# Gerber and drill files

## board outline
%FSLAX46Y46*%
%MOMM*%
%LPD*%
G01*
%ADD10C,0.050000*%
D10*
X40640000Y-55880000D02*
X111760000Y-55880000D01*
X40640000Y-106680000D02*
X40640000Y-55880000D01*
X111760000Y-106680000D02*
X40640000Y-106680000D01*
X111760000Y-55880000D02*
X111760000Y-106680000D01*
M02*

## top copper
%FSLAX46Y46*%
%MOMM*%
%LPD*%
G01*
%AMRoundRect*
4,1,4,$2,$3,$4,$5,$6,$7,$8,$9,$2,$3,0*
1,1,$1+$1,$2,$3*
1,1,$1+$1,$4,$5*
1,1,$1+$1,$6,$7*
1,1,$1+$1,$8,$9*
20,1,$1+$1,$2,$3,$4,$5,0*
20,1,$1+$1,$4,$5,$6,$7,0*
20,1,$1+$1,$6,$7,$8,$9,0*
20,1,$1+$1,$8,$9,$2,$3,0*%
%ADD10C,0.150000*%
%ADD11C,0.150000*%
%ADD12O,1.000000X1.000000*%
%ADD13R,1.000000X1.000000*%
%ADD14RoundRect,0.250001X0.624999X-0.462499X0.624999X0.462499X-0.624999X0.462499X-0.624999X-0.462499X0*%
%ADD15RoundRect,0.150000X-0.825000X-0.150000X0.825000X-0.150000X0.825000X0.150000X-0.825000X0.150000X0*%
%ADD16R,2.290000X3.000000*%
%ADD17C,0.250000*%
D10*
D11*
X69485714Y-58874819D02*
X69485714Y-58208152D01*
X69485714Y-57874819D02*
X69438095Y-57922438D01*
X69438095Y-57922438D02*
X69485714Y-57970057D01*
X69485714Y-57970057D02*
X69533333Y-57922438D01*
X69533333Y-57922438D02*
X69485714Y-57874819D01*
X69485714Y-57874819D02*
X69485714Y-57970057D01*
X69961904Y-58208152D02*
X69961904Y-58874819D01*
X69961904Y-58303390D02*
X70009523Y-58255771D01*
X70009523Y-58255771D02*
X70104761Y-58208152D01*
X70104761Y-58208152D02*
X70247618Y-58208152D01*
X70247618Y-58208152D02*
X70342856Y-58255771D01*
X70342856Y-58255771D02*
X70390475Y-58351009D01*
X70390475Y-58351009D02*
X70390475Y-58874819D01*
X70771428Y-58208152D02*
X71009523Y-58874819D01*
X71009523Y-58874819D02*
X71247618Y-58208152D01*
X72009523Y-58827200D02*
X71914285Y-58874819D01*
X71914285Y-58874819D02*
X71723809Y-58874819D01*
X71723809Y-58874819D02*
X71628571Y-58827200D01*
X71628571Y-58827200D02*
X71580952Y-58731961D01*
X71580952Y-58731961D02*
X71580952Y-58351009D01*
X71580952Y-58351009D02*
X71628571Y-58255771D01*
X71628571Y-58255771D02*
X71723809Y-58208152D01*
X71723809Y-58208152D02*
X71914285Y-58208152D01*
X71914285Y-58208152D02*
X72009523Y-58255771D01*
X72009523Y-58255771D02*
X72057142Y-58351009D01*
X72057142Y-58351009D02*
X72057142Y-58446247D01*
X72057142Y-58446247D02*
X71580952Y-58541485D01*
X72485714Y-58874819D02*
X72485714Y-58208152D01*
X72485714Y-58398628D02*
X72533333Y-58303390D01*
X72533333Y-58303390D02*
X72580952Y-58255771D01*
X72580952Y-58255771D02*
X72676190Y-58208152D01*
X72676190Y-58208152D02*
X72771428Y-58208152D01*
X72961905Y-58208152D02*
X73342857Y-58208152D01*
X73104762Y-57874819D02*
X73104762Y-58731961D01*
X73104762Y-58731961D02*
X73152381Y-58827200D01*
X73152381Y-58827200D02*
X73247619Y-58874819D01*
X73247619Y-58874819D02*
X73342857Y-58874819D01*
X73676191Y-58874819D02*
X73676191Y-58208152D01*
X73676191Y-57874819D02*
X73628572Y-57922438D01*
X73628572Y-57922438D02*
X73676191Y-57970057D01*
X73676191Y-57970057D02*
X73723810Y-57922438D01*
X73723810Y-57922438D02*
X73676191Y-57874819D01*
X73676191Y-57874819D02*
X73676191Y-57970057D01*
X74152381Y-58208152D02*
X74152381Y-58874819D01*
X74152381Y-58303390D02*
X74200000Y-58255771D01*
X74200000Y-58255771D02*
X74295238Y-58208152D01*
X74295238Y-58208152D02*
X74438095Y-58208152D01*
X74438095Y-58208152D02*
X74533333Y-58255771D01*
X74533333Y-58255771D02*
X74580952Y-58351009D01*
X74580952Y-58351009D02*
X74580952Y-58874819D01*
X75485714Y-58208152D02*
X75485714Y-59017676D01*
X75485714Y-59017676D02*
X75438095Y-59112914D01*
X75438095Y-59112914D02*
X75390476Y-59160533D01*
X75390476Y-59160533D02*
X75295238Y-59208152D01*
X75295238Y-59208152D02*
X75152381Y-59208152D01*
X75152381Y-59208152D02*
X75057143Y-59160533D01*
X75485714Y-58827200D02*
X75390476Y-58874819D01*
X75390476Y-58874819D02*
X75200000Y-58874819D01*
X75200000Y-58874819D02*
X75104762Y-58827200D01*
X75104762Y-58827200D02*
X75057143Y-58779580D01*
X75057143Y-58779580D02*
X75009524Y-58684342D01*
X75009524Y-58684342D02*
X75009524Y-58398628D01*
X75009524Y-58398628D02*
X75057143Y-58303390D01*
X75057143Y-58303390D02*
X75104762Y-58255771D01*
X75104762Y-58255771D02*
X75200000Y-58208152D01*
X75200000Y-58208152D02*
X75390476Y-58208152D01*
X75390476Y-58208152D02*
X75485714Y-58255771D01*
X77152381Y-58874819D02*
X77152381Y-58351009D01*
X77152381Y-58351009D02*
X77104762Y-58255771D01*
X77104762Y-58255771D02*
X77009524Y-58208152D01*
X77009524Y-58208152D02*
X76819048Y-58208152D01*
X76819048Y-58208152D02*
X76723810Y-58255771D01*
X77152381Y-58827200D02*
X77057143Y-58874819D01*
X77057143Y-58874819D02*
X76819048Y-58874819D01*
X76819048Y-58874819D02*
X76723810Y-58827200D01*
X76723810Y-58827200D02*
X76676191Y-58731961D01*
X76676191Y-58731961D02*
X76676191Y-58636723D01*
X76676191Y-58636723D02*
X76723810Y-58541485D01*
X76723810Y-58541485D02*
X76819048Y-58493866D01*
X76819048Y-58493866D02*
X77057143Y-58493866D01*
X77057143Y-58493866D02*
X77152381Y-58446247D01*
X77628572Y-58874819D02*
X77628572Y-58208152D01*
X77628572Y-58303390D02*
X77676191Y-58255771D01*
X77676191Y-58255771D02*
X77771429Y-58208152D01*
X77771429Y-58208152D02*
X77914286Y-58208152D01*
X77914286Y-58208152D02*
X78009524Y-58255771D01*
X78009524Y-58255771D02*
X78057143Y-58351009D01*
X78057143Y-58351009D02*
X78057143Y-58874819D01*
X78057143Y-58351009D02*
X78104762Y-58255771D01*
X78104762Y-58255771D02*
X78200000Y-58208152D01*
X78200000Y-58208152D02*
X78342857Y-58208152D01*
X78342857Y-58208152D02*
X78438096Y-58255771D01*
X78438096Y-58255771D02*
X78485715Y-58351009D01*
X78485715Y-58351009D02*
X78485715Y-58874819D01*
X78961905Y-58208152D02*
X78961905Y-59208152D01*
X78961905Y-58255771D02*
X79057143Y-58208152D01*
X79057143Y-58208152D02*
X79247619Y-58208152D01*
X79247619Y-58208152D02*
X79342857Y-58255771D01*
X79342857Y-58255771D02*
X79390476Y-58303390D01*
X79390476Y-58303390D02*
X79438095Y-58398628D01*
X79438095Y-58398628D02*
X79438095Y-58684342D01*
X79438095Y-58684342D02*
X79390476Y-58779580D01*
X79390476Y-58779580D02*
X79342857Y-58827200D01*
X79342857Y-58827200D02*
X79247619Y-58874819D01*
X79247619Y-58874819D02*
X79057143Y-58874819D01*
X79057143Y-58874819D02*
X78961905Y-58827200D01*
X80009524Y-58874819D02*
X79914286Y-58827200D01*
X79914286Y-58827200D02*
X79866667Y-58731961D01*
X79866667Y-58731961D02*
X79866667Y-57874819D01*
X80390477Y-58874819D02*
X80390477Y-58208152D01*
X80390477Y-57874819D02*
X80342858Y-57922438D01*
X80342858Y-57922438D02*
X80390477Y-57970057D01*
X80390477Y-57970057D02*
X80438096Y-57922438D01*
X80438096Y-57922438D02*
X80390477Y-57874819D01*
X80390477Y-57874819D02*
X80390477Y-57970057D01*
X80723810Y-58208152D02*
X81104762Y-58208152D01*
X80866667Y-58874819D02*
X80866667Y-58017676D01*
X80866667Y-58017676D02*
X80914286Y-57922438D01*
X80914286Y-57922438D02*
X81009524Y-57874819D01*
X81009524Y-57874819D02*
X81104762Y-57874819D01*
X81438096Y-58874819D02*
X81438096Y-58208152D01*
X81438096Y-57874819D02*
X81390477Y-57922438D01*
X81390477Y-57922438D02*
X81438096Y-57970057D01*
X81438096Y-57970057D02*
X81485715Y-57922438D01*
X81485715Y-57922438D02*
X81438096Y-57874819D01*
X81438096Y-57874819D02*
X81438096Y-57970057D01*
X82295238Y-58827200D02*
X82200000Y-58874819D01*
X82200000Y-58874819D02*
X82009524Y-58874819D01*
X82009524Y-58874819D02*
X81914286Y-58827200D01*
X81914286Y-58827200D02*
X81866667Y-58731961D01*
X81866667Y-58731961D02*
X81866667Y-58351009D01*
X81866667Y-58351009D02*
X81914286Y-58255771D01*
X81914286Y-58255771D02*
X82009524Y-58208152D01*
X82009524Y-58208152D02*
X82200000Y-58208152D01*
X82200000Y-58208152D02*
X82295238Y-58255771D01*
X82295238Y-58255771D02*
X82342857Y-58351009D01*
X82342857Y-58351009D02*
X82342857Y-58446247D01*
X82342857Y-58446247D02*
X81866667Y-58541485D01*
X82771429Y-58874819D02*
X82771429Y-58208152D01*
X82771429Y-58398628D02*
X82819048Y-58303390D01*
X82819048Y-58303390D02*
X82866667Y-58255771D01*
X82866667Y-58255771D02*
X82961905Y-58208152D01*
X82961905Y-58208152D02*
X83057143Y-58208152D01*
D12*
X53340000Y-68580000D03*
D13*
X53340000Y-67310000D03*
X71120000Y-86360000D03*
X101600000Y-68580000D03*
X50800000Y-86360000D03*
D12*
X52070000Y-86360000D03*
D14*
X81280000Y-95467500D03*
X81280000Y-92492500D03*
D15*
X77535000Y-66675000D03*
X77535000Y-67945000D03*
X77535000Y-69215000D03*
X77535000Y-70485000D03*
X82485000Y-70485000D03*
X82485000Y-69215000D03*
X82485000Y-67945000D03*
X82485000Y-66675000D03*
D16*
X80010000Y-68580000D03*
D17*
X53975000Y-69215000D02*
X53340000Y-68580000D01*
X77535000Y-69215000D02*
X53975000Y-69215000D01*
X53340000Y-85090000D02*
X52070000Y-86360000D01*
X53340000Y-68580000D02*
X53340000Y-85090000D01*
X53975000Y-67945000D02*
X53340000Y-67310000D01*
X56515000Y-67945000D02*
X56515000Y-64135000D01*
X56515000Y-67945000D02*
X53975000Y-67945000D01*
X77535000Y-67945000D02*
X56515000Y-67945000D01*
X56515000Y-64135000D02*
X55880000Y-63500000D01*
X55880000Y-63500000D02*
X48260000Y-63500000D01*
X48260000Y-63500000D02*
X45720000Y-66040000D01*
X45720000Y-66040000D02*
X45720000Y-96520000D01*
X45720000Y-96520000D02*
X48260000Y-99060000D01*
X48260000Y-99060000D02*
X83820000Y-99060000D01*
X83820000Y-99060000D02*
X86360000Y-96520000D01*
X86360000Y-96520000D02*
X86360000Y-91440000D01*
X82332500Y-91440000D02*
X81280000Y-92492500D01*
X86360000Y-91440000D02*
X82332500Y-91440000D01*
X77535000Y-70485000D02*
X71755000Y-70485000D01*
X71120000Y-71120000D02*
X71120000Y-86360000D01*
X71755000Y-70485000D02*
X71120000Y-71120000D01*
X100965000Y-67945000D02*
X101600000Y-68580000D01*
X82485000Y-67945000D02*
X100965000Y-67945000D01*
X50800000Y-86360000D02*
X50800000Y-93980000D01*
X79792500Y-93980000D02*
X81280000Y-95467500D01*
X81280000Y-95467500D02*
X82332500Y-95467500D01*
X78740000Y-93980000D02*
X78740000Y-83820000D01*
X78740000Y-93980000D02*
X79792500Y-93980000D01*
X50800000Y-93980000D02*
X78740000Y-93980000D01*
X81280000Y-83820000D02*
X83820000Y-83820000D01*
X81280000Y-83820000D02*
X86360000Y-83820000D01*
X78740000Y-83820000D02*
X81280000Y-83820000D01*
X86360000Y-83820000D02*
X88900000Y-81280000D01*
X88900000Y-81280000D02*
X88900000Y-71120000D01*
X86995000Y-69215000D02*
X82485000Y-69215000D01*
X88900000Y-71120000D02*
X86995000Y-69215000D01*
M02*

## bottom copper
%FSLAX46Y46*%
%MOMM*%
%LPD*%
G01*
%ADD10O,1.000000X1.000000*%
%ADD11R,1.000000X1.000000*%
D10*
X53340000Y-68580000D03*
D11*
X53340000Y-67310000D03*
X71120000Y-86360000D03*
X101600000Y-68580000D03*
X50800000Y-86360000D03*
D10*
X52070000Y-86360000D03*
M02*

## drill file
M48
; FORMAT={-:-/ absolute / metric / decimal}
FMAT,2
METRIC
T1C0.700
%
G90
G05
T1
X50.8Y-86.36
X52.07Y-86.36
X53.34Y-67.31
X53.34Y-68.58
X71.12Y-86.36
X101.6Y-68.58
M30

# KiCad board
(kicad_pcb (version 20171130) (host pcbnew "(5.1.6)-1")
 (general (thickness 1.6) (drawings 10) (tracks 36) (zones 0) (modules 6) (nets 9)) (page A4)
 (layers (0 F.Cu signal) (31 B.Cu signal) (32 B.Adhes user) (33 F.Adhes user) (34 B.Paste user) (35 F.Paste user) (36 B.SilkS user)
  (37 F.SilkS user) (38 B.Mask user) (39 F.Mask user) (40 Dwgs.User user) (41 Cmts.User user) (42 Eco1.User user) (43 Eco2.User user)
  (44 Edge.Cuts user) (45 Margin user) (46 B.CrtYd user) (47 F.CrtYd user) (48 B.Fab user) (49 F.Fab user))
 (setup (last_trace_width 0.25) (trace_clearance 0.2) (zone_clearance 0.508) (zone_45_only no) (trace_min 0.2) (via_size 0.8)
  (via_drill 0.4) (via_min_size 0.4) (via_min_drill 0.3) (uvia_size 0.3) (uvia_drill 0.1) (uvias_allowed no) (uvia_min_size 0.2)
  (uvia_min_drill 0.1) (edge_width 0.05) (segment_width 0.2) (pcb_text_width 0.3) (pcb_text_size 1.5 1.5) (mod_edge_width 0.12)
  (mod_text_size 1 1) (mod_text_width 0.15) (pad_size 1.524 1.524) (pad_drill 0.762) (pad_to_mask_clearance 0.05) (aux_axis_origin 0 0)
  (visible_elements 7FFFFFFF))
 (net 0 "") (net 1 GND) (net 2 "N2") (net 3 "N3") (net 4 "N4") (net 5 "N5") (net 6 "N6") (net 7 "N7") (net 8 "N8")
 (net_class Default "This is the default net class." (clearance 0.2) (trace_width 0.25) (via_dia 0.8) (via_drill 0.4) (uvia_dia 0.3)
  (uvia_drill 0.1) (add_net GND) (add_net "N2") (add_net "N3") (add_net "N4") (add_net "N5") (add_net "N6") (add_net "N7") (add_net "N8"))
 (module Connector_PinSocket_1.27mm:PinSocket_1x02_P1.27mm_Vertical (layer F.Cu) (at 53.34 67.31)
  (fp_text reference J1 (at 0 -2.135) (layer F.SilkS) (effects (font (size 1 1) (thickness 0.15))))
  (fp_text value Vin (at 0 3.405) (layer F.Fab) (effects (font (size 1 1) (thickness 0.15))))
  (pad 2 thru_hole oval (at 0 1.27) (size 1 1) (drill 0.7) (layers *.Cu *.Mask) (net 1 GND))
  (pad 1 thru_hole rect (at 0 0) (size 1 1) (drill 0.7) (layers *.Cu *.Mask) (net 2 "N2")))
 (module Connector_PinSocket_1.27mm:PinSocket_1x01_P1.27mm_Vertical (layer F.Cu) (at 71.12 86.36)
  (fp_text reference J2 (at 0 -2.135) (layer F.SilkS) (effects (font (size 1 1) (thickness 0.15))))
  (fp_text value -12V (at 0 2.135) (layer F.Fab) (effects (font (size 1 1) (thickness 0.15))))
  (pad 1 thru_hole rect (at 0 0) (size 1 1) (drill 0.7) (layers *.Cu *.Mask) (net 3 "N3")))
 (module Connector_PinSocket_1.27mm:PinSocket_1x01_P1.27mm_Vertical (layer F.Cu) (at 101.6 68.58)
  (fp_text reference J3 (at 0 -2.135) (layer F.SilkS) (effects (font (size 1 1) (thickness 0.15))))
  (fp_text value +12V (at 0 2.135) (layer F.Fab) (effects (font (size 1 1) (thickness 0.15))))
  (pad 1 thru_hole rect (at 0 0) (size 1 1) (drill 0.7) (layers *.Cu *.Mask) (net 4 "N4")))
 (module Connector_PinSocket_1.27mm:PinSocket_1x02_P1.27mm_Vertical (layer F.Cu) (at 50.8 86.36 90)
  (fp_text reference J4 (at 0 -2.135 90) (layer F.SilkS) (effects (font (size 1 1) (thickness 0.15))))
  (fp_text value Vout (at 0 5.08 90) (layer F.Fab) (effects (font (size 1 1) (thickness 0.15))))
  (pad 1 thru_hole rect (at 0 0 90) (size 1 1) (drill 0.7) (layers *.Cu *.Mask) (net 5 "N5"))
  (pad 2 thru_hole oval (at 0 1.27 90) (size 1 1) (drill 0.7) (layers *.Cu *.Mask) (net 1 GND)))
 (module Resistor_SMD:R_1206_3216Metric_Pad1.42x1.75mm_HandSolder (layer F.Cu) (at 81.28 93.98 90)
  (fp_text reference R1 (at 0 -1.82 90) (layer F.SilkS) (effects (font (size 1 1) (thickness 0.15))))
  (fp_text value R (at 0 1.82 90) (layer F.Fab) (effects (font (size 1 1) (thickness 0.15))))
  (pad 1 smd roundrect (at -1.4875 0 90) (size 1.425 1.75) (layers F.Cu F.Paste F.Mask) (roundrect_rratio 0.175439) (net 5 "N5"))
  (pad 2 smd roundrect (at 1.4875 0 90) (size 1.425 1.75) (layers F.Cu F.Paste F.Mask) (roundrect_rratio 0.175439) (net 2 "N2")))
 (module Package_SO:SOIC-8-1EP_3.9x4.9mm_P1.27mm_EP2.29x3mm (layer F.Cu) (at 80.01 68.58)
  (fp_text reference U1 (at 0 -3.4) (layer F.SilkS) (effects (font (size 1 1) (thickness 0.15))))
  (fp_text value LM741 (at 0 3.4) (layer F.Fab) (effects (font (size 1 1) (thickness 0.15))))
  (pad 1 smd roundrect (at -2.475 -1.905) (size 1.95 0.6) (layers F.Cu F.Paste F.Mask) (roundrect_rratio 0.25) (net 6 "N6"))
  (pad 2 smd roundrect (at -2.475 -0.635) (size 1.95 0.6) (layers F.Cu F.Paste F.Mask) (roundrect_rratio 0.25) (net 2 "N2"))
  (pad 3 smd roundrect (at -2.475 0.635) (size 1.95 0.6) (layers F.Cu F.Paste F.Mask) (roundrect_rratio 0.25) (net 1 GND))
  (pad 4 smd roundrect (at -2.475 1.905) (size 1.95 0.6) (layers F.Cu F.Paste F.Mask) (roundrect_rratio 0.25) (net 3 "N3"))
  (pad 5 smd roundrect (at 2.475 1.905) (size 1.95 0.6) (layers F.Cu F.Paste F.Mask) (roundrect_rratio 0.25) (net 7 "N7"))
  (pad 6 smd roundrect (at 2.475 0.635) (size 1.95 0.6) (layers F.Cu F.Paste F.Mask) (roundrect_rratio 0.25) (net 5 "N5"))
  (pad 7 smd roundrect (at 2.475 -0.635) (size 1.95 0.6) (layers F.Cu F.Paste F.Mask) (roundrect_rratio 0.25) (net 4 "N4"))
  (pad 8 smd roundrect (at 2.475 -1.905) (size 1.95 0.6) (layers F.Cu F.Paste F.Mask) (roundrect_rratio 0.25) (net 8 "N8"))
  (pad 9 smd rect (at 0 0) (size 2.29 3) (layers F.Cu F.Mask))
  (pad "" smd roundrect (at -0.57 -0.75) (size 0.92 1.21) (layers F.Paste) (roundrect_rratio 0.25))
  (pad "" smd roundrect (at -0.57 0.75) (size 0.92 1.21) (layers F.Paste) (roundrect_rratio 0.25))
  (pad "" smd roundrect (at 0.57 -0.75) (size 0.92 1.21) (layers F.Paste) (roundrect_rratio 0.25))
  (pad "" smd roundrect (at 0.57 0.75) (size 0.92 1.21) (layers F.Paste) (roundrect_rratio 0.25)))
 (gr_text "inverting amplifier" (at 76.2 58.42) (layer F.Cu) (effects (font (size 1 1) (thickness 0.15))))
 (gr_line (start 40.64 55.88) (end 111.76 55.88) (layer Edge.Cuts) (width 0.05))
 (gr_line (start 40.64 106.68) (end 40.64 55.88) (layer Edge.Cuts) (width 0.05))
 (gr_line (start 111.76 106.68) (end 40.64 106.68) (layer Edge.Cuts) (width 0.05))
 (gr_line (start 111.76 55.88) (end 111.76 106.68) (layer Edge.Cuts) (width 0.05))
 (segment (start 53.975 69.215) (end 53.34 68.58) (width 0.25) (layer F.Cu) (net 1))
 (segment (start 77.535 69.215) (end 53.975 69.215) (width 0.25) (layer F.Cu) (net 1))
 (segment (start 53.34 85.09) (end 52.07 86.36) (width 0.25) (layer F.Cu) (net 1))
 (segment (start 53.34 68.58) (end 53.34 85.09) (width 0.25) (layer F.Cu) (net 1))
 (segment (start 53.975 67.945) (end 53.34 67.31) (width 0.25) (layer F.Cu) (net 2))
 (segment (start 56.515 67.945) (end 56.515 64.135) (width 0.25) (layer F.Cu) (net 2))
 (segment (start 56.515 67.945) (end 53.975 67.945) (width 0.25) (layer F.Cu) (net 2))
 (segment (start 77.535 67.945) (end 56.515 67.945) (width 0.25) (layer F.Cu) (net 2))
 (segment (start 56.515 64.135) (end 55.88 63.5) (width 0.25) (layer F.Cu) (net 2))
 (segment (start 55.88 63.5) (end 48.26 63.5) (width 0.25) (layer F.Cu) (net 2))
 (segment (start 48.26 63.5) (end 45.72 66.04) (width 0.25) (layer F.Cu) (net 2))
 (segment (start 45.72 66.04) (end 45.72 96.52) (width 0.25) (layer F.Cu) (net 2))
 (segment (start 45.72 96.52) (end 48.26 99.06) (width 0.25) (layer F.Cu) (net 2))
 (segment (start 48.26 99.06) (end 83.82 99.06) (width 0.25) (layer F.Cu) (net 2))
 (segment (start 83.82 99.06) (end 86.36 96.52) (width 0.25) (layer F.Cu) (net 2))
 (segment (start 86.36 96.52) (end 86.36 91.44) (width 0.25) (layer F.Cu) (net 2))
 (segment (start 82.3325 91.44) (end 81.28 92.4925) (width 0.25) (layer F.Cu) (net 2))
 (segment (start 86.36 91.44) (end 82.3325 91.44) (width 0.25) (layer F.Cu) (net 2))
 (segment (start 77.535 70.485) (end 71.755 70.485) (width 0.25) (layer F.Cu) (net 3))
 (segment (start 71.12 71.12) (end 71.12 86.36) (width 0.25) (layer F.Cu) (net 3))
 (segment (start 71.755 70.485) (end 71.12 71.12) (width 0.25) (layer F.Cu) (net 3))
 (segment (start 100.965 67.945) (end 101.6 68.58) (width 0.25) (layer F.Cu) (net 4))
 (segment (start 82.485 67.945) (end 100.965 67.945) (width 0.25) (layer F.Cu) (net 4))
 (segment (start 50.8 86.36) (end 50.8 93.98) (width 0.25) (layer F.Cu) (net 5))
 (segment (start 79.7925 93.98) (end 81.28 95.4675) (width 0.25) (layer F.Cu) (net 5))
 (segment (start 81.28 95.4675) (end 82.3325 95.4675) (width 0.25) (layer F.Cu) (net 5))
 (segment (start 78.74 93.98) (end 78.74 83.82) (width 0.25) (layer F.Cu) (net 5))
 (segment (start 78.74 93.98) (end 79.7925 93.98) (width 0.25) (layer F.Cu) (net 5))
 (segment (start 50.8 93.98) (end 78.74 93.98) (width 0.25) (layer F.Cu) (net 5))
 (segment (start 81.28 83.82) (end 83.82 83.82) (width 0.25) (layer F.Cu) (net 5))
 (segment (start 81.28 83.82) (end 86.36 83.82) (width 0.25) (layer F.Cu) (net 5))
 (segment (start 78.74 83.82) (end 81.28 83.82) (width 0.25) (layer F.Cu) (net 5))
 (segment (start 86.36 83.82) (end 88.9 81.28) (width 0.25) (layer F.Cu) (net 5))
 (segment (start 88.9 81.28) (end 88.9 71.12) (width 0.25) (layer F.Cu) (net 5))
 (segment (start 86.995 69.215) (end 82.485 69.215) (width 0.25) (layer F.Cu) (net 5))
 (segment (start 88.9 71.12) (end 86.995 69.215) (width 0.25) (layer F.Cu) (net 5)))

